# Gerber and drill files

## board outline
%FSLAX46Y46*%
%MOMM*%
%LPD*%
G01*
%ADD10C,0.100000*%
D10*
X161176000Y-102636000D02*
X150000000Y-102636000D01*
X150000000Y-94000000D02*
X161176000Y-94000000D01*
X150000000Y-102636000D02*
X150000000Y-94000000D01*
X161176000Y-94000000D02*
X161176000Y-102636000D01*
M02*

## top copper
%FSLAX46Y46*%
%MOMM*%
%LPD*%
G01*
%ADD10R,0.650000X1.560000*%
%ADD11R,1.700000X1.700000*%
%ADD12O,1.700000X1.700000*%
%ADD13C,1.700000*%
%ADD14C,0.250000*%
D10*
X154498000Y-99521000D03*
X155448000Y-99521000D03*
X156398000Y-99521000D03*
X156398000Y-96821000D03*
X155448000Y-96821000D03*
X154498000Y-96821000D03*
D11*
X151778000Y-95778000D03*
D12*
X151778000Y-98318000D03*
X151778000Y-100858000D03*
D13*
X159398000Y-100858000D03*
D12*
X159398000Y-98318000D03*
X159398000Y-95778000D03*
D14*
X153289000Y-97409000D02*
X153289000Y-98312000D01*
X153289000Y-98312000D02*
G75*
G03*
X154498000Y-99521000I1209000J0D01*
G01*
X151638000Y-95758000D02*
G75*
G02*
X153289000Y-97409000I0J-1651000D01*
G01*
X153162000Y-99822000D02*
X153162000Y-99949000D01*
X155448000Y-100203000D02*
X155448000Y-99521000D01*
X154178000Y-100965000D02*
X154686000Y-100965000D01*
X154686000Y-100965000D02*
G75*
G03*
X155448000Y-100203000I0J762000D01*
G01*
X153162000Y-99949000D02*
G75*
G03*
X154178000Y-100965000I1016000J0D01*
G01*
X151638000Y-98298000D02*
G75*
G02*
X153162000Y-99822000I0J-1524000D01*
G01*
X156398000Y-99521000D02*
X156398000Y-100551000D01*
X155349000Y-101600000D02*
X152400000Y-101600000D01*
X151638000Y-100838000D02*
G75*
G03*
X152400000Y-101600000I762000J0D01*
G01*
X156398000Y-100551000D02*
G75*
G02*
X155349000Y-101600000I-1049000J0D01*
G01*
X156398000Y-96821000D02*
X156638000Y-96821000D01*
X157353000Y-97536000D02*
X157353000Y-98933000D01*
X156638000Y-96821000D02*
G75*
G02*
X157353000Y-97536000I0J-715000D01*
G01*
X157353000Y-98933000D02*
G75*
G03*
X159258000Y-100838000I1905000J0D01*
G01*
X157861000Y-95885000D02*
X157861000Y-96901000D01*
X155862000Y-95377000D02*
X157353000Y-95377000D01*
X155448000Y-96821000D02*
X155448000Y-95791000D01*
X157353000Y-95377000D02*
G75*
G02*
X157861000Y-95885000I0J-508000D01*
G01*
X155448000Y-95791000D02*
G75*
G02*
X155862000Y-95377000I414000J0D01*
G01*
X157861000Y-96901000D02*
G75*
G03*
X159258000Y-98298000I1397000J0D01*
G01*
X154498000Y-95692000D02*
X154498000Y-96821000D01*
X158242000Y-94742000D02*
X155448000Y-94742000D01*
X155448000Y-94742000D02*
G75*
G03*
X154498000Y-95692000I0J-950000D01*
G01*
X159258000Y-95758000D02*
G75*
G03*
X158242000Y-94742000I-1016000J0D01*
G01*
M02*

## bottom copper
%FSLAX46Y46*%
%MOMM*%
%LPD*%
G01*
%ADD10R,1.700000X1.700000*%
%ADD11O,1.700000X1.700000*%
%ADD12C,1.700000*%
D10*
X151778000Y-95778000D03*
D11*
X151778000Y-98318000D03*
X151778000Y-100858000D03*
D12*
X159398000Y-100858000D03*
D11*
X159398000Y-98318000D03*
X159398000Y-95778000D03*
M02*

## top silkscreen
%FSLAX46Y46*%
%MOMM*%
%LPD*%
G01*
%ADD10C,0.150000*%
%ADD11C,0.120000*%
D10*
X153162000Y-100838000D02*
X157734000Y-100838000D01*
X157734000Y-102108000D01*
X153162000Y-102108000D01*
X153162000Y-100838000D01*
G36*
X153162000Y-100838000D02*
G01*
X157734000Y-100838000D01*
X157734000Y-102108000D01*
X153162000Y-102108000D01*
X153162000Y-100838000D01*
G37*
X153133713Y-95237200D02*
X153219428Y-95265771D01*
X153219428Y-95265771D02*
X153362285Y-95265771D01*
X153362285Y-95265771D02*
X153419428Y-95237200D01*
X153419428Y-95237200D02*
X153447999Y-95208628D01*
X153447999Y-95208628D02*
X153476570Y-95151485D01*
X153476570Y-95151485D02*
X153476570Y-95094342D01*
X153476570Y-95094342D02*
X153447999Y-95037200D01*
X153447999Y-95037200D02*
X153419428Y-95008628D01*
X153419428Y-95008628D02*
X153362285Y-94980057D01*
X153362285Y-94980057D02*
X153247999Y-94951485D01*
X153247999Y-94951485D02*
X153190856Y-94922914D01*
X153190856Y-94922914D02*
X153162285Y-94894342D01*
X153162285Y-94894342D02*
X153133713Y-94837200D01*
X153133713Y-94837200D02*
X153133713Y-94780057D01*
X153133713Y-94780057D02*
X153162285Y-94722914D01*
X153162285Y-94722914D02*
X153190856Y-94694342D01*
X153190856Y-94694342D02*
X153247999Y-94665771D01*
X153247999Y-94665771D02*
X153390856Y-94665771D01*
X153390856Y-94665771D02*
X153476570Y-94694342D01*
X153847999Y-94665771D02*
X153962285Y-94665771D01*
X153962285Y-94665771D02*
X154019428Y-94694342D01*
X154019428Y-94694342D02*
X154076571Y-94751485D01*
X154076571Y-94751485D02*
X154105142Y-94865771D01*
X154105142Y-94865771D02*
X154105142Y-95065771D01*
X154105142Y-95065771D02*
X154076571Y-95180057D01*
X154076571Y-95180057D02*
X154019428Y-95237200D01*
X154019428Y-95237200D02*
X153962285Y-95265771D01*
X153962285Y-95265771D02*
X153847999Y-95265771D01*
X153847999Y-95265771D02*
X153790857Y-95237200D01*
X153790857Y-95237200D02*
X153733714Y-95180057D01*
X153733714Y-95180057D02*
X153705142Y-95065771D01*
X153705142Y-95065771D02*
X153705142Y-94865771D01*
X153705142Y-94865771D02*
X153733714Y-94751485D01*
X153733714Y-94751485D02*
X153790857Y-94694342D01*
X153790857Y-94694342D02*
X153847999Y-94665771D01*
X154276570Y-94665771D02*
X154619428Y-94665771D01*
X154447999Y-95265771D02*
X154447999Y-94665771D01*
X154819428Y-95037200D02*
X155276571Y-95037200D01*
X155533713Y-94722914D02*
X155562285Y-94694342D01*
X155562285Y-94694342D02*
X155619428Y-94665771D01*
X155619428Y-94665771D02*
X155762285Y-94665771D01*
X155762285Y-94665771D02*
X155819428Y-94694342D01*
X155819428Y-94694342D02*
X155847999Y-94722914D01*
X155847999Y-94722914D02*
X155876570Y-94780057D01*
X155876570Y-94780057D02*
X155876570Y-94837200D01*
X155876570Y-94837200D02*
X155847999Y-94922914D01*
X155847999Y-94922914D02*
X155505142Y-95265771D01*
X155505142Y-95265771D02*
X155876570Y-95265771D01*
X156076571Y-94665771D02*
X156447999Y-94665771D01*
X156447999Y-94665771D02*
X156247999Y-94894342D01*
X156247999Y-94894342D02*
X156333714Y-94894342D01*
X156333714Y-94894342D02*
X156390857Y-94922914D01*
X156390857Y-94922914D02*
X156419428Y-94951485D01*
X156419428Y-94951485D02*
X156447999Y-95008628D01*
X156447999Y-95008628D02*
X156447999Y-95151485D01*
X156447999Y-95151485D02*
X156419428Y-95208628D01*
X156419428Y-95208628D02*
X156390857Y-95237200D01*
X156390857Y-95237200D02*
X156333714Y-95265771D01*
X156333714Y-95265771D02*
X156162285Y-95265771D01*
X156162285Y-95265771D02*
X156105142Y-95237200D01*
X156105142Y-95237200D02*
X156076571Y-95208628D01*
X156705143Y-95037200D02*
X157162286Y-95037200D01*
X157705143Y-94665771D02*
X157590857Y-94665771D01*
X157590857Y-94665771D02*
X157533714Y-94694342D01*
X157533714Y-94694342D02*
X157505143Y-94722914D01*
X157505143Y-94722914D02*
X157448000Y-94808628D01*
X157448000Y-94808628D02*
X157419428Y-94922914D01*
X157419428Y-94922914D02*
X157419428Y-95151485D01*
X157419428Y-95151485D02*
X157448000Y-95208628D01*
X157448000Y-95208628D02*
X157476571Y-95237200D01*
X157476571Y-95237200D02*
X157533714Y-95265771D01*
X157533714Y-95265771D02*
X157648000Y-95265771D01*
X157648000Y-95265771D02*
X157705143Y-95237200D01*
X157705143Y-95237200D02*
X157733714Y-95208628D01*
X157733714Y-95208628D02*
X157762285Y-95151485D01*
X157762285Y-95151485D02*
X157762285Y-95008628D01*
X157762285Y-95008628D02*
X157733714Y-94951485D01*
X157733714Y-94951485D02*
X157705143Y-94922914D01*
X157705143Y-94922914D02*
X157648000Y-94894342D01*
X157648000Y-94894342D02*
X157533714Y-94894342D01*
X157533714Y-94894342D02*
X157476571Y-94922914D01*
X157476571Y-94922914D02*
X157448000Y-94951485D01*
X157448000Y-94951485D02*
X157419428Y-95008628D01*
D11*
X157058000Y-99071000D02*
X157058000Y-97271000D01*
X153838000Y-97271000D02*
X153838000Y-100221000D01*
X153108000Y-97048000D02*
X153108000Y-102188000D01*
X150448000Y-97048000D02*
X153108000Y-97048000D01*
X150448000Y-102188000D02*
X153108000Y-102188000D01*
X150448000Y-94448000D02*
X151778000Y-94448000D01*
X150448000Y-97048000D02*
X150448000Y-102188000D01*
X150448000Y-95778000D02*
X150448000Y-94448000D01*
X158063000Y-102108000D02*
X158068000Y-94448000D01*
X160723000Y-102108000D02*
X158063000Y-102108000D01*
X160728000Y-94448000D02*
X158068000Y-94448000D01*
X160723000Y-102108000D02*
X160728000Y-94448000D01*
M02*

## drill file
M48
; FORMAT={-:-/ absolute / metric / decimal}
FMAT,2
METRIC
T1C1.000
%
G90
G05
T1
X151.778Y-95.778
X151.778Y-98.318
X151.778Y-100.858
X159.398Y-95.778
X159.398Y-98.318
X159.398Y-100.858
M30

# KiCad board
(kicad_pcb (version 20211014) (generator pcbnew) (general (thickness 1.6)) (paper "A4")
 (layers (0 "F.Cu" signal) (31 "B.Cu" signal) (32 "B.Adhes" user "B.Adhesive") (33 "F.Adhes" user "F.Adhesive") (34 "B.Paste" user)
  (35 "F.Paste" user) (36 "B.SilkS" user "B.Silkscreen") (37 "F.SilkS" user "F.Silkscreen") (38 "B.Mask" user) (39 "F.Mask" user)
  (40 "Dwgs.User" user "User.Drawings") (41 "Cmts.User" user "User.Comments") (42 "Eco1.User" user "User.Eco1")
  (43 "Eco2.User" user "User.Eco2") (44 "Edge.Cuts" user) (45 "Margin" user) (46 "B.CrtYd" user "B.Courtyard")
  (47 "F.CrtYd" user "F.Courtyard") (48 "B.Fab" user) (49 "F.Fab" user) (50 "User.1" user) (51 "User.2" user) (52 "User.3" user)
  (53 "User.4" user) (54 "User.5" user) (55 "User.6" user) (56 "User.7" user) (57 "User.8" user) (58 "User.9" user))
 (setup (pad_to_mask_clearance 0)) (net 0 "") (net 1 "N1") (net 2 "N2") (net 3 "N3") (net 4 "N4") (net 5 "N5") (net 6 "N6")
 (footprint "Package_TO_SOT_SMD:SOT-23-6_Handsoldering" (layer "F.Cu") (at 155.448 98.171 90)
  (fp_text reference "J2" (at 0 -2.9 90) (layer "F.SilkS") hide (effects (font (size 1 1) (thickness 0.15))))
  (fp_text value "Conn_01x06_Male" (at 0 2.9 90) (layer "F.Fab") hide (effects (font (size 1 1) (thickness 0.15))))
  (fp_line (start -0.9 1.61) (end 0.9 1.61) (layer "F.SilkS") (width 0.12))
  (fp_line (start 0.9 -1.61) (end -2.05 -1.61) (layer "F.SilkS") (width 0.12))
  (pad "1" smd rect (at -1.35 -0.95 90) (size 1.56 0.65) (layers "F.Cu" "F.Paste" "F.Mask") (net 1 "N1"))
  (pad "2" smd rect (at -1.35 0 90) (size 1.56 0.65) (layers "F.Cu" "F.Paste" "F.Mask") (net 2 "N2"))
  (pad "3" smd rect (at -1.35 0.95 90) (size 1.56 0.65) (layers "F.Cu" "F.Paste" "F.Mask") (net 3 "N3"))
  (pad "4" smd rect (at 1.35 0.95 90) (size 1.56 0.65) (layers "F.Cu" "F.Paste" "F.Mask") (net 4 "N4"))
  (pad "5" smd rect (at 1.35 0 90) (size 1.56 0.65) (layers "F.Cu" "F.Paste" "F.Mask") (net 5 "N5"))
  (pad "6" smd rect (at 1.35 -0.95 90) (size 1.56 0.65) (layers "F.Cu" "F.Paste" "F.Mask") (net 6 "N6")))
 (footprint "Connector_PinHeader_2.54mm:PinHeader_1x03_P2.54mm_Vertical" (layer "F.Cu") (at 151.778 95.778)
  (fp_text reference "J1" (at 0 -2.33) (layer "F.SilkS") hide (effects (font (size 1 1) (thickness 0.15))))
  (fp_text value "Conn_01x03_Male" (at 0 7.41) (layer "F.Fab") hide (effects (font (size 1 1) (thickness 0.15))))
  (fp_line (start 1.33 1.27) (end 1.33 6.41) (layer "F.SilkS") (width 0.12))
  (fp_line (start -1.33 1.27) (end 1.33 1.27) (layer "F.SilkS") (width 0.12))
  (fp_line (start -1.33 6.41) (end 1.33 6.41) (layer "F.SilkS") (width 0.12))
  (fp_line (start -1.33 -1.33) (end 0 -1.33) (layer "F.SilkS") (width 0.12))
  (fp_line (start -1.33 1.27) (end -1.33 6.41) (layer "F.SilkS") (width 0.12))
  (fp_line (start -1.33 0) (end -1.33 -1.33) (layer "F.SilkS") (width 0.12))
  (pad "1" thru_hole rect (at 0 0) (size 1.7 1.7) (drill 1) (layers *.Cu *.Mask) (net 1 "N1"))
  (pad "2" thru_hole oval (at 0 2.54) (size 1.7 1.7) (drill 1) (layers *.Cu *.Mask) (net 2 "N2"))
  (pad "3" thru_hole oval (at 0 5.08) (size 1.7 1.7) (drill 1) (layers *.Cu *.Mask) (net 3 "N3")))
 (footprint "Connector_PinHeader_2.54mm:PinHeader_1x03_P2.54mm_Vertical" (layer "F.Cu") (at 159.398 100.858 180)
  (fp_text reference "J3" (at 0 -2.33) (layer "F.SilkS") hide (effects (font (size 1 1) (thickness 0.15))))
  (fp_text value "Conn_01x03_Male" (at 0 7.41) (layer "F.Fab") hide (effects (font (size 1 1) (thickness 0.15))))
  (fp_line (start 1.335 -1.25) (end 1.33 6.41) (layer "F.SilkS") (width 0.12))
  (fp_line (start -1.325 -1.25) (end 1.335 -1.25) (layer "F.SilkS") (width 0.12))
  (fp_line (start -1.33 6.41) (end 1.33 6.41) (layer "F.SilkS") (width 0.12))
  (fp_line (start -1.325 -1.25) (end -1.33 6.41) (layer "F.SilkS") (width 0.12))
  (pad "1" thru_hole circle (at 0 0 180) (size 1.7 1.7) (drill 1) (layers *.Cu *.Mask) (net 4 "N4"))
  (pad "2" thru_hole oval (at 0 2.54 180) (size 1.7 1.7) (drill 1) (layers *.Cu *.Mask) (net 5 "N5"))
  (pad "3" thru_hole oval (at 0 5.08 180) (size 1.7 1.7) (drill 1) (layers *.Cu *.Mask) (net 6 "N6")))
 (gr_rect (start 153.162 100.838) (end 157.734 102.108) (layer "F.SilkS") (width 0.15) (fill solid))
 (gr_line (start 161.176 102.636) (end 150 102.636) (layer "Edge.Cuts") (width 0.1))
 (gr_line (start 150 94) (end 161.176 94) (layer "Edge.Cuts") (width 0.1))
 (gr_line (start 150 102.636) (end 150 94) (layer "Edge.Cuts") (width 0.1))
 (gr_line (start 161.176 94) (end 161.176 102.636) (layer "Edge.Cuts") (width 0.1))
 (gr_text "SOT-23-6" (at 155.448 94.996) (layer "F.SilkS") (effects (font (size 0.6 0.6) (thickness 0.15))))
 (segment (start 153.289 97.409) (end 153.289 98.312) (width 0.25) (layer "F.Cu") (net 1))
 (arc (start 153.289 98.312) (mid 153.643108 99.166892) (end 154.498 99.521) (width 0.25) (layer "F.Cu") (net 1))
 (arc (start 151.638 95.758) (mid 152.805433 96.241567) (end 153.289 97.409) (width 0.25) (layer "F.Cu") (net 1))
 (segment (start 153.162 99.822) (end 153.162 99.949) (width 0.25) (layer "F.Cu") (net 2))
 (segment (start 155.448 100.203) (end 155.448 99.521) (width 0.25) (layer "F.Cu") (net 2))
 (segment (start 154.178 100.965) (end 154.686 100.965) (width 0.25) (layer "F.Cu") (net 2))
 (arc (start 154.686 100.965) (mid 155.224815 100.741815) (end 155.448 100.203) (width 0.25) (layer "F.Cu") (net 2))
 (arc (start 153.162 99.949) (mid 153.45958 100.66742) (end 154.178 100.965) (width 0.25) (layer "F.Cu") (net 2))
 (arc (start 151.638 98.298) (mid 152.715631 98.744369) (end 153.162 99.822) (width 0.25) (layer "F.Cu") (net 2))
 (segment (start 156.398 99.521) (end 156.398 100.551) (width 0.25) (layer "F.Cu") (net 3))
 (segment (start 155.349 101.6) (end 152.4 101.6) (width 0.25) (layer "F.Cu") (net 3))
 (arc (start 151.638 100.838) (mid 151.861185 101.376815) (end 152.4 101.6) (width 0.25) (layer "F.Cu") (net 3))
 (arc (start 156.398 100.551) (mid 156.090755 101.292755) (end 155.349 101.6) (width 0.25) (layer "F.Cu") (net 3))
 (segment (start 156.398 96.821) (end 156.638 96.821) (width 0.25) (layer "F.Cu") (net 4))
 (segment (start 157.353 97.536) (end 157.353 98.933) (width 0.25) (layer "F.Cu") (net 4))
 (arc (start 156.638 96.821) (mid 157.143581 97.030419) (end 157.353 97.536) (width 0.25) (layer "F.Cu") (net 4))
 (arc (start 157.353 98.933) (mid 157.910962 100.280038) (end 159.258 100.838) (width 0.25) (layer "F.Cu") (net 4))
 (segment (start 157.861 95.885) (end 157.861 96.901) (width 0.25) (layer "F.Cu") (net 5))
 (segment (start 155.862 95.377) (end 157.353 95.377) (width 0.25) (layer "F.Cu") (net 5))
 (segment (start 155.448 96.821) (end 155.448 95.791) (width 0.25) (layer "F.Cu") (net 5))
 (arc (start 157.353 95.377) (mid 157.71221 95.52579) (end 157.861 95.885) (width 0.25) (layer "F.Cu") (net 5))
 (arc (start 155.448 95.791) (mid 155.569258 95.498258) (end 155.862 95.377) (width 0.25) (layer "F.Cu") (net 5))
 (arc (start 157.861 96.901) (mid 158.270172 97.888828) (end 159.258 98.298) (width 0.25) (layer "F.Cu") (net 5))
 (segment (start 154.498 95.692) (end 154.498 96.821) (width 0.25) (layer "F.Cu") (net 6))
 (segment (start 158.242 94.742) (end 155.448 94.742) (width 0.25) (layer "F.Cu") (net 6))
 (arc (start 155.448 94.742) (mid 154.776249 95.020249) (end 154.498 95.692) (width 0.25) (layer "F.Cu") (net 6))
 (arc (start 159.258 95.758) (mid 158.96042 95.03958) (end 158.242 94.742) (width 0.25) (layer "F.Cu") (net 6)))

